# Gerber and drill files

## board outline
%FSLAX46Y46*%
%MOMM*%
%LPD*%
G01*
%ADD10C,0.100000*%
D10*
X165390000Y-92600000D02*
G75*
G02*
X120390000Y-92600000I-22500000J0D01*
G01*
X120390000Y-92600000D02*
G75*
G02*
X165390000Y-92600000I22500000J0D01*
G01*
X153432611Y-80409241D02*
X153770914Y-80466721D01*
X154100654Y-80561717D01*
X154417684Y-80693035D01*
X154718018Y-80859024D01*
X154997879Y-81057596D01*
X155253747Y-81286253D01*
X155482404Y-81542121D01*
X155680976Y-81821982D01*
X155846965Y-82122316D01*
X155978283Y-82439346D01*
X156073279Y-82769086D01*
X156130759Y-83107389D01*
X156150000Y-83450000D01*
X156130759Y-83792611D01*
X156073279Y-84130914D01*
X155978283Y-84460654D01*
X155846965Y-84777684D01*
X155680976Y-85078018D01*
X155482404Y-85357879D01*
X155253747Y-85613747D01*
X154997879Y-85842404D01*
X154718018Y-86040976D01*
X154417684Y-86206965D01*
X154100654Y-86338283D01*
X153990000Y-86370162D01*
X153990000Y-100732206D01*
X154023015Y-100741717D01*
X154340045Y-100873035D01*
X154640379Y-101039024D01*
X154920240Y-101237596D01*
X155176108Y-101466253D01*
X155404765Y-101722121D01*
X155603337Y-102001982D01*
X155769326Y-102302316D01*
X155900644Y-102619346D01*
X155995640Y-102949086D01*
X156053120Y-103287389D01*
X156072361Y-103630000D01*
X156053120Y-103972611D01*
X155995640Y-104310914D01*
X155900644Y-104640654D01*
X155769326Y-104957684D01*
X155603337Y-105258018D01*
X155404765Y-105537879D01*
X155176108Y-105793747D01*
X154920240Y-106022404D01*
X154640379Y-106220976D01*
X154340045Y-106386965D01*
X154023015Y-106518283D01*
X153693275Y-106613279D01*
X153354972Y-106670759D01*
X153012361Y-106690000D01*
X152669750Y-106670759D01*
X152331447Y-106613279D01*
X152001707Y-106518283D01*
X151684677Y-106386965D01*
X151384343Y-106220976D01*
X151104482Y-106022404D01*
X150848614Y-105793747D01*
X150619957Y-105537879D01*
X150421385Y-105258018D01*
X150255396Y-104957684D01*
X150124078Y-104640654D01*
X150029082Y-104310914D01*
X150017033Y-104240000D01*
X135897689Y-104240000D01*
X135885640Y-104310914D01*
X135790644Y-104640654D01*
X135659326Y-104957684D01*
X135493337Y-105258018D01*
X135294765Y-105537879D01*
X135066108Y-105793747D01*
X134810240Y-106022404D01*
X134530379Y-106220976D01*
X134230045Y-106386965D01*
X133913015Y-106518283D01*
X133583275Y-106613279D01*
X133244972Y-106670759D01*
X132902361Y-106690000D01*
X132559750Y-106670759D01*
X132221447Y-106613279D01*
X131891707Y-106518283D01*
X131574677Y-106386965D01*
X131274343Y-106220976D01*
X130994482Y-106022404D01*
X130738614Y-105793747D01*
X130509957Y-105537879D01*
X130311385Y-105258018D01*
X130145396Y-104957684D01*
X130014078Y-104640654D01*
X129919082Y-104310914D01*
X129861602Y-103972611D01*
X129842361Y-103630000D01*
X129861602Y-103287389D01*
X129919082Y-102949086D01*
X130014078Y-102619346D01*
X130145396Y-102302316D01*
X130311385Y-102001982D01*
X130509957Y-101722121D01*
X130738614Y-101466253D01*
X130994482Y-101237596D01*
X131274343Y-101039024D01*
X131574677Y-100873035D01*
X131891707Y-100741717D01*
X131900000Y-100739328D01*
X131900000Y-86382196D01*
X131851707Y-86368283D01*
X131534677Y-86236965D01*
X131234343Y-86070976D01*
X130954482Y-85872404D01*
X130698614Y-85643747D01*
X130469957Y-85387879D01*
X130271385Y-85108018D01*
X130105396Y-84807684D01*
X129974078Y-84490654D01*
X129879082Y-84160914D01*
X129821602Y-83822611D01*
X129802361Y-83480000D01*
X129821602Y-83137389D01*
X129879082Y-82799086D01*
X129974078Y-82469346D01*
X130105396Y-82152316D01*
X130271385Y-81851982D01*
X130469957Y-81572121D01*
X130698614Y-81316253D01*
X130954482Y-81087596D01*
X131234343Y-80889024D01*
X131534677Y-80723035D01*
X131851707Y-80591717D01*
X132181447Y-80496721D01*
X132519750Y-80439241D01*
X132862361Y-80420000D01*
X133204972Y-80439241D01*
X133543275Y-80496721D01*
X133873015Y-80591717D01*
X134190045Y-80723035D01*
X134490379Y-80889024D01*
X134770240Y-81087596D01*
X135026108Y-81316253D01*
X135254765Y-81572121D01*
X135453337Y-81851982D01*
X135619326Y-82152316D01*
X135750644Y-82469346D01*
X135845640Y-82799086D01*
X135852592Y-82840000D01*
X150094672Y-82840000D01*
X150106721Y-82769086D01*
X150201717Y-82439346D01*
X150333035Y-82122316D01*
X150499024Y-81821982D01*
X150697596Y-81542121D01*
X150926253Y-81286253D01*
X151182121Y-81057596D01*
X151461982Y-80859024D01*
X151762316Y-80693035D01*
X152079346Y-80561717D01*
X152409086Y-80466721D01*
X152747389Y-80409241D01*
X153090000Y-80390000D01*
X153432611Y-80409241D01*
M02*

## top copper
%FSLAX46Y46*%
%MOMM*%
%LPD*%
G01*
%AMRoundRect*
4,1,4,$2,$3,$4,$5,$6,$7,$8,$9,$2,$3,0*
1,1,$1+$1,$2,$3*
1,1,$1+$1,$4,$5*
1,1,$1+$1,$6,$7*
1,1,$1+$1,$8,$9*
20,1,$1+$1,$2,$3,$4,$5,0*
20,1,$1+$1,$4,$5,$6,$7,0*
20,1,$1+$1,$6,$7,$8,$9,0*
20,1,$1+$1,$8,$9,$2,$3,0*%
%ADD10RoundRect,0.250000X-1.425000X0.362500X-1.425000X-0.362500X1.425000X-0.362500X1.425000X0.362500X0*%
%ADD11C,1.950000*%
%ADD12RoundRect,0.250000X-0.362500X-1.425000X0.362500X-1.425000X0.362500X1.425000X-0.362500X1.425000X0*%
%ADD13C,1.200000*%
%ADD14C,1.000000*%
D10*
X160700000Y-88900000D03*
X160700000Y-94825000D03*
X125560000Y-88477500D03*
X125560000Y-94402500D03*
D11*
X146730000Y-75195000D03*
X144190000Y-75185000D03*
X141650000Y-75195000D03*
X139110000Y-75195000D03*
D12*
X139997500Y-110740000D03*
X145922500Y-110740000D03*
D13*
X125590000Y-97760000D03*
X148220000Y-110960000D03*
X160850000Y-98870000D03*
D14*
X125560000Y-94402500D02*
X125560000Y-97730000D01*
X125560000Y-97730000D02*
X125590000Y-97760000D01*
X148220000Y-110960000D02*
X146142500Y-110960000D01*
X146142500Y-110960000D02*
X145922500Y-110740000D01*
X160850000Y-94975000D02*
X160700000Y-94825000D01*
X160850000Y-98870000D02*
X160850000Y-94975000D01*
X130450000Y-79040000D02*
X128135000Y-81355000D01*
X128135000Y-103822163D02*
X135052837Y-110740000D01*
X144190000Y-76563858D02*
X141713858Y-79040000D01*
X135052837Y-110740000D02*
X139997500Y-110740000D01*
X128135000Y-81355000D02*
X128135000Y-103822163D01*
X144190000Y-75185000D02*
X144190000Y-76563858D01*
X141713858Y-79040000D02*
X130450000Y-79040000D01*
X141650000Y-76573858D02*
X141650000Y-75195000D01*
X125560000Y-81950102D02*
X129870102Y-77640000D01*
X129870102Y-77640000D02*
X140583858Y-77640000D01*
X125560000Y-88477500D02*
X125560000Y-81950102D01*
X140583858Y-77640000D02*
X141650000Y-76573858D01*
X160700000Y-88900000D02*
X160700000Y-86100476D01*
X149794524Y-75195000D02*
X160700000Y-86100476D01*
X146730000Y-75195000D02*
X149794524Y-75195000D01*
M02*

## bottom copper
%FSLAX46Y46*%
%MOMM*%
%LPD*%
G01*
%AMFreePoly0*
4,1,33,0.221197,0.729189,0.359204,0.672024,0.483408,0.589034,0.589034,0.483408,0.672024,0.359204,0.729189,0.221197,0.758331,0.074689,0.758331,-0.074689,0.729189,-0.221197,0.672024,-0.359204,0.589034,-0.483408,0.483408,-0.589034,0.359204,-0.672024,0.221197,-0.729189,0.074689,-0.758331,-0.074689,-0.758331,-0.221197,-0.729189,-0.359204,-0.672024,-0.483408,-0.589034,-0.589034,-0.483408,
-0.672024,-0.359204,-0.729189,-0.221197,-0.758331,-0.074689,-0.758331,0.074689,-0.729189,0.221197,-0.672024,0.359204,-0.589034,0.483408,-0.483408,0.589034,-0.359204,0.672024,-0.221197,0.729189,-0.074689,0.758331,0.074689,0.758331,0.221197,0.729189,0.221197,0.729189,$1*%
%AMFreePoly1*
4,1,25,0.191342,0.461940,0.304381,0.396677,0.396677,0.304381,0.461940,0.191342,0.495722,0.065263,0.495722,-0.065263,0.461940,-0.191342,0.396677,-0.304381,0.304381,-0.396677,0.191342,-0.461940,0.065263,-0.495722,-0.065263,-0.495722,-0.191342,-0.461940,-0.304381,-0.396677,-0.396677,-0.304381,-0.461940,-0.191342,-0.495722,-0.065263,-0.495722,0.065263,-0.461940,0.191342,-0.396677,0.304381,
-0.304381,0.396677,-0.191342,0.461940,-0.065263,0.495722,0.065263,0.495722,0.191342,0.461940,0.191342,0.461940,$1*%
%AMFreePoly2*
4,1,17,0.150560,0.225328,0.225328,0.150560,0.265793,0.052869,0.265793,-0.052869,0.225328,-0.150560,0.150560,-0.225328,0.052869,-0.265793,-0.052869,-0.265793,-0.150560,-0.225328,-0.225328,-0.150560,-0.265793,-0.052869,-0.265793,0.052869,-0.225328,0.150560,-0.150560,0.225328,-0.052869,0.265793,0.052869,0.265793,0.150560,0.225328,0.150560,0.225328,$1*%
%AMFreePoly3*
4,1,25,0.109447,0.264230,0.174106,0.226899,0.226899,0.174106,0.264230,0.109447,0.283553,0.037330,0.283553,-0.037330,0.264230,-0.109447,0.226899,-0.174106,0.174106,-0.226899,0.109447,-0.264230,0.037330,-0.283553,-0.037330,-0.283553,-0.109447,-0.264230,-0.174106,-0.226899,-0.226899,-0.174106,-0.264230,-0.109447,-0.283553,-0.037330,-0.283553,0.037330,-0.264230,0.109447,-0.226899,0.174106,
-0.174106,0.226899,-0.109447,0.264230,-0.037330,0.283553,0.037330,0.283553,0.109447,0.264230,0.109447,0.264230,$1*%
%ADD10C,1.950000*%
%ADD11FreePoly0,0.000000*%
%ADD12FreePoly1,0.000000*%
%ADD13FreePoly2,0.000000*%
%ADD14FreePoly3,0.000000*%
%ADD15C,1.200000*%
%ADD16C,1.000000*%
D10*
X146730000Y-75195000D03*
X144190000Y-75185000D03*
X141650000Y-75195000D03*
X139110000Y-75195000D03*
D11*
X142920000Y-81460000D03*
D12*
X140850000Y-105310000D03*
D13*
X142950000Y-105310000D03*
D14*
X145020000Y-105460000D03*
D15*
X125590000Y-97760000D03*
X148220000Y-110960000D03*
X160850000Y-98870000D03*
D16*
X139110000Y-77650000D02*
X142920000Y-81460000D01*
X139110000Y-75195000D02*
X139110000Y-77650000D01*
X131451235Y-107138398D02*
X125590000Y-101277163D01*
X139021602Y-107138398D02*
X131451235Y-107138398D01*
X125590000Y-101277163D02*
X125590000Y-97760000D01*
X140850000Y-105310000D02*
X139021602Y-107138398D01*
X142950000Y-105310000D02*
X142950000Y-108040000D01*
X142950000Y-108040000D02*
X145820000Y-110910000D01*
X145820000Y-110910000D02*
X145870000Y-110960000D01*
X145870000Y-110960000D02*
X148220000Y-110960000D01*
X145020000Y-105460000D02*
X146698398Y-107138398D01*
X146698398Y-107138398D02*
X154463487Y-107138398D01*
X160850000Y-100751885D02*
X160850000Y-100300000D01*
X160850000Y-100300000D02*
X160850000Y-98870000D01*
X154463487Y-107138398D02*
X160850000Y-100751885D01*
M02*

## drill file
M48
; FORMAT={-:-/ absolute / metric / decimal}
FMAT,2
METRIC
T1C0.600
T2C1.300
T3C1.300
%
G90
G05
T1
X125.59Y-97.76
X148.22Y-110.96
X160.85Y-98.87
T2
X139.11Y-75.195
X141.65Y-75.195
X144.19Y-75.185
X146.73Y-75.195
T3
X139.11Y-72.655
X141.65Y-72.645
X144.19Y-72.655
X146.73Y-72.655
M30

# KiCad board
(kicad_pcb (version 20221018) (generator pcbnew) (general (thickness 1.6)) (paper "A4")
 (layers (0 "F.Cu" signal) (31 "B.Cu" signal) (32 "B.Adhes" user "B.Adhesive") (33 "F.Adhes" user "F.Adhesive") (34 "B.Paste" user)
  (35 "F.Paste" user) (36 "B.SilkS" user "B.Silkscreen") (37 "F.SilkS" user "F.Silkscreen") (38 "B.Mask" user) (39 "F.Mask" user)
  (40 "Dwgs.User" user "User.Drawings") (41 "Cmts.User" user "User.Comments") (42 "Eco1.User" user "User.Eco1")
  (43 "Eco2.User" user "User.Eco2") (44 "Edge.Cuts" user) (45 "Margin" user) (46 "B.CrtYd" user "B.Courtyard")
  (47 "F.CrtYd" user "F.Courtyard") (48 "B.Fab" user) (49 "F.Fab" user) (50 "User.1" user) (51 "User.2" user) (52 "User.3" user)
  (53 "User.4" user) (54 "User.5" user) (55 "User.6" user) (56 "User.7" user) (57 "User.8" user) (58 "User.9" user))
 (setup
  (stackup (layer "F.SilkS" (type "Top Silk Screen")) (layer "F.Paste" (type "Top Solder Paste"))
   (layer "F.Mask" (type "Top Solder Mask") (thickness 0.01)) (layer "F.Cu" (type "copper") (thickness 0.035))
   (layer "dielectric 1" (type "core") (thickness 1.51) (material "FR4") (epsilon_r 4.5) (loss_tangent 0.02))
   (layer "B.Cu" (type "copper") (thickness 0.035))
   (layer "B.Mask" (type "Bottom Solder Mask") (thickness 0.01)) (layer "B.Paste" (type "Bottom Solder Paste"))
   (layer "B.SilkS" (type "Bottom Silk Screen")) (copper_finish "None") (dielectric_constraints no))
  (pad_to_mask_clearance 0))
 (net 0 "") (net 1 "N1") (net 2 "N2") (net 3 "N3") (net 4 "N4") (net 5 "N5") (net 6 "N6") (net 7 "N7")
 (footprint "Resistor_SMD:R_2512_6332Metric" (layer "F.Cu") (at 160.7 91.8625 -90)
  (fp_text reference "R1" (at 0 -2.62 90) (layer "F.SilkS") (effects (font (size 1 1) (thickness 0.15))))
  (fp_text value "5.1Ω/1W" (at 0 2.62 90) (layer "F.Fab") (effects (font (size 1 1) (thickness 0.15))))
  (pad "1" smd roundrect (at -2.9625 0 270) (size 1.225 3.35) (layers "F.Cu" "F.Paste" "F.Mask") (roundrect_rratio 0.2040816327)
   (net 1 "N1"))
  (pad "2" smd roundrect (at 2.9625 0 270) (size 1.225 3.35) (layers "F.Cu" "F.Paste" "F.Mask") (roundrect_rratio 0.2040816327) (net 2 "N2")))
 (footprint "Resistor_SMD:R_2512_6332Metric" (layer "F.Cu") (at 125.56 91.44 -90)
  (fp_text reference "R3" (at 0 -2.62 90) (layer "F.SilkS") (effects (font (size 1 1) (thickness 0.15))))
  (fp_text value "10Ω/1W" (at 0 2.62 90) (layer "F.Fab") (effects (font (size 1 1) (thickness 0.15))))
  (pad "1" smd roundrect (at -2.9625 0 270) (size 1.225 3.35) (layers "F.Cu" "F.Paste" "F.Mask") (roundrect_rratio 0.2040816327)
   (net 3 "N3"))
  (pad "2" smd roundrect (at 2.9625 0 270) (size 1.225 3.35) (layers "F.Cu" "F.Paste" "F.Mask") (roundrect_rratio 0.2040816327) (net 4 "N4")))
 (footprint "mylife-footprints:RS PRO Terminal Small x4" (layer "F.Cu") (at 146.73 75.195 180)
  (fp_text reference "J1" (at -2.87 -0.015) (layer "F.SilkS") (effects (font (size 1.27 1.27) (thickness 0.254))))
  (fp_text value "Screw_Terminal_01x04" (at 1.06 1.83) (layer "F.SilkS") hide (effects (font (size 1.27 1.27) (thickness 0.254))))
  (pad "" np_thru_hole circle (at 0 2.54 180) (size 1.3 1.3) (drill 1.3) (layers "*.Cu" "*.Mask"))
  (pad "" np_thru_hole circle (at 2.54 2.54 180) (size 1.3 1.3) (drill 1.3) (layers "*.Cu" "*.Mask"))
  (pad "" np_thru_hole circle (at 5.08 2.55 180) (size 1.3 1.3) (drill 1.3) (layers "*.Cu" "*.Mask"))
  (pad "" np_thru_hole circle (at 7.62 2.54 180) (size 1.3 1.3) (drill 1.3) (layers "*.Cu" "*.Mask"))
  (pad "1" thru_hole circle (at 0 0 180) (size 1.95 1.95) (drill 1.3) (layers "*.Cu" "*.Mask") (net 1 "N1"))
  (pad "2" thru_hole circle (at 2.54 0.01 180) (size 1.95 1.95) (drill 1.3) (layers "*.Cu" "*.Mask") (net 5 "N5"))
  (pad "3" thru_hole circle (at 5.08 0 180) (size 1.95 1.95) (drill 1.3) (layers "*.Cu" "*.Mask") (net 3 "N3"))
  (pad "4" thru_hole circle (at 7.62 0 180) (size 1.95 1.95) (drill 1.3) (layers "*.Cu" "*.Mask") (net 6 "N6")))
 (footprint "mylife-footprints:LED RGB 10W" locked (layer "F.Cu") (at 142.94 92.59)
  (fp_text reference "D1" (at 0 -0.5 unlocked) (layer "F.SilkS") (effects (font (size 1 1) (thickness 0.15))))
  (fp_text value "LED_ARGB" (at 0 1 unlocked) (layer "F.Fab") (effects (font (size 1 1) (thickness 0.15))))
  (fp_poly
   (pts (xy 10.492611 -12.180759) (xy 10.830914 -12.123279) (xy 11.160654 -12.028283) (xy 11.477684 -11.896965) (xy 11.778018 -11.730976)
    (xy 12.057879 -11.532404) (xy 12.313747 -11.303747) (xy 12.542404 -11.047879) (xy 12.740976 -10.768018) (xy 12.906965 -10.467684)
    (xy 13.038283 -10.150654) (xy 13.133279 -9.820914) (xy 13.190759 -9.482611) (xy 13.21 -9.14) (xy 13.190759 -8.797389)
    (xy 13.133279 -8.459086) (xy 13.038283 -8.129346) (xy 12.906965 -7.812316) (xy 12.740976 -7.511982) (xy 12.542404 -7.232121)
    (xy 12.313747 -6.976253) (xy 12.057879 -6.747596) (xy 11.778018 -6.549024) (xy 11.477684 -6.383035) (xy 11.160654 -6.251717)
    (xy 11.05 -6.219838) (xy 11.05 8.142206) (xy 11.083015 8.151717) (xy 11.400045 8.283035) (xy 11.700379 8.449024) (xy 11.98024 8.647596)
    (xy 12.236108 8.876253) (xy 12.464765 9.132121) (xy 12.663337 9.411982) (xy 12.829326 9.712316) (xy 12.960644 10.029346)
    (xy 13.05564 10.359086) (xy 13.11312 10.697389) (xy 13.132361 11.04) (xy 13.11312 11.382611) (xy 13.05564 11.720914)
    (xy 12.960644 12.050654) (xy 12.829326 12.367684) (xy 12.663337 12.668018) (xy 12.464765 12.947879) (xy 12.236108 13.203747)
    (xy 11.98024 13.432404) (xy 11.700379 13.630976) (xy 11.400045 13.796965) (xy 11.083015 13.928283) (xy 10.753275 14.023279)
    (xy 10.414972 14.080759) (xy 10.072361 14.1) (xy 9.72975 14.080759) (xy 9.391447 14.023279) (xy 9.061707 13.928283)
    (xy 8.744677 13.796965) (xy 8.444343 13.630976) (xy 8.164482 13.432404) (xy 7.908614 13.203747) (xy 7.679957 12.947879)
    (xy 7.481385 12.668018) (xy 7.315396 12.367684) (xy 7.184078 12.050654) (xy 7.089082 11.720914) (xy 7.077033 11.65) (xy -7.042311 11.65)
    (xy -7.05436 11.720914) (xy -7.149356 12.050654) (xy -7.280674 12.367684) (xy -7.446663 12.668018) (xy -7.645235 12.947879)
    (xy -7.873892 13.203747) (xy -8.12976 13.432404) (xy -8.409621 13.630976) (xy -8.709955 13.796965) (xy -9.026985 13.928283)
    (xy -9.356725 14.023279) (xy -9.695028 14.080759) (xy -10.037639 14.1) (xy -10.38025 14.080759) (xy -10.718553 14.023279)
    (xy -11.048293 13.928283) (xy -11.365323 13.796965) (xy -11.665657 13.630976) (xy -11.945518 13.432404) (xy -12.201386 13.203747)
    (xy -12.430043 12.947879) (xy -12.628615 12.668018) (xy -12.794604 12.367684) (xy -12.925922 12.050654) (xy -13.020918 11.720914)
    (xy -13.078398 11.382611) (xy -13.097639 11.04) (xy -13.078398 10.697389) (xy -13.020918 10.359086) (xy -12.925922 10.029346)
    (xy -12.794604 9.712316) (xy -12.628615 9.411982) (xy -12.430043 9.132121) (xy -12.201386 8.876253) (xy -11.945518 8.647596)
    (xy -11.665657 8.449024) (xy -11.365323 8.283035) (xy -11.048293 8.151717) (xy -11.04 8.149328) (xy -11.04 -6.207804)
    (xy -11.088293 -6.221717) (xy -11.405323 -6.353035) (xy -11.705657 -6.519024) (xy -11.985518 -6.717596) (xy -12.241386 -6.946253)
    (xy -12.470043 -7.202121) (xy -12.668615 -7.481982) (xy -12.834604 -7.782316) (xy -12.965922 -8.099346) (xy -13.060918 -8.429086)
    (xy -13.118398 -8.767389) (xy -13.137639 -9.11) (xy -13.118398 -9.452611) (xy -13.060918 -9.790914) (xy -12.965922 -10.120654)
    (xy -12.834604 -10.437684) (xy -12.668615 -10.738018) (xy -12.470043 -11.017879) (xy -12.241386 -11.273747) (xy -11.985518 -11.502404)
    (xy -11.705657 -11.700976) (xy -11.405323 -11.866965) (xy -11.088293 -11.998283) (xy -10.758553 -12.093279) (xy -10.42025 -12.150759)
    (xy -10.077639 -12.17) (xy -9.735028 -12.150759) (xy -9.396725 -12.093279) (xy -9.066985 -11.998283) (xy -8.749955 -11.866965)
    (xy -8.449621 -11.700976) (xy -8.16976 -11.502404) (xy -7.913892 -11.273747) (xy -7.685235 -11.017879) (xy -7.486663 -10.738018)
    (xy -7.320674 -10.437684) (xy -7.189356 -10.120654) (xy -7.09436 -9.790914) (xy -7.087408 -9.75) (xy 7.154672 -9.75)
    (xy 7.166721 -9.820914) (xy 7.261717 -10.150654) (xy 7.393035 -10.467684) (xy 7.559024 -10.768018) (xy 7.757596 -11.047879)
    (xy 7.986253 -11.303747) (xy 8.242121 -11.532404) (xy 8.521982 -11.730976) (xy 8.822316 -11.896965) (xy 9.139346 -12.028283)
    (xy 9.469086 -12.123279) (xy 9.807389 -12.180759) (xy 10.15 -12.2))
   (stroke (width 0.1) (type solid)) (fill none) (layer "Edge.Cuts"))
  (pad "1" smd custom locked (at -0.02 -11.13) (size 1.524 1.524) (layers "B.Cu" "B.Paste" "B.Mask") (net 6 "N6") (thermal_bridge_angle 45)
   (options (clearance outline) (anchor circle)) (primitives))
  (pad "2" smd custom locked (at -2.09 12.72) (size 1 1) (layers "B.Cu" "B.Paste" "B.Mask") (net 4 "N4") (thermal_bridge_angle 45)
   (options (clearance outline) (anchor circle)) (primitives))
  (pad "3" smd custom locked (at 0.01 12.72) (size 0.542 0.542) (layers "B.Cu" "B.Paste" "B.Mask") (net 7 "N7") (thermal_bridge_angle 45)
   (options (clearance outline) (anchor circle)) (primitives))
  (pad "4" smd custom locked (at 2.08 12.87) (size 0.572 0.572) (layers "B.Cu" "B.Paste" "B.Mask") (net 2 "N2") (thermal_bridge_angle 45)
   (options (clearance outline) (anchor circle)) (primitives)))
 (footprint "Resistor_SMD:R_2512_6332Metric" (layer "F.Cu") (at 142.96 110.74)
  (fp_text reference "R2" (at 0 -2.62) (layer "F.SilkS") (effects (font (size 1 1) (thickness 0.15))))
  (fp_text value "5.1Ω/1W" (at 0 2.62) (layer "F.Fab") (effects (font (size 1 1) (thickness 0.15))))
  (pad "1" smd roundrect (at -2.9625 0) (size 1.225 3.35) (layers "F.Cu" "F.Paste" "F.Mask") (roundrect_rratio 0.2040816327) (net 5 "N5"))
  (pad "2" smd roundrect (at 2.9625 0) (size 1.225 3.35) (layers "F.Cu" "F.Paste" "F.Mask") (roundrect_rratio 0.2040816327) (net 7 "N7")))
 (gr_circle locked (center 142.89 92.6) (end 165.39 92.6) (stroke (width 0.1) (type default)) (fill none) (layer "Edge.Cuts"))
 (segment (start 139.11 77.65) (end 142.92 81.46) (width 1) (layer "B.Cu") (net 6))
 (segment (start 139.11 75.195) (end 139.11 77.65) (width 1) (layer "B.Cu") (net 6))
 (segment (start 125.56 94.4025) (end 125.56 97.73) (width 1) (layer "F.Cu") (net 4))
 (segment (start 125.56 97.73) (end 125.59 97.76) (width 1) (layer "F.Cu") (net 4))
 (via (at 125.59 97.76) (size 1.2) (drill 0.6) (layers "F.Cu" "B.Cu") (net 4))
 (segment (start 131.451235 107.138398) (end 125.59 101.277163) (width 1) (layer "B.Cu") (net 4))
 (segment (start 139.021602 107.138398) (end 131.451235 107.138398) (width 1) (layer "B.Cu") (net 4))
 (segment (start 125.59 101.277163) (end 125.59 97.76) (width 1) (layer "B.Cu") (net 4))
 (segment (start 140.85 105.31) (end 139.021602 107.138398) (width 1) (layer "B.Cu") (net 4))
 (segment (start 148.22 110.96) (end 146.1425 110.96) (width 1) (layer "F.Cu") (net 7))
 (segment (start 146.1425 110.96) (end 145.9225 110.74) (width 1) (layer "F.Cu") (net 7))
 (via (at 148.22 110.96) (size 1.2) (drill 0.6) (layers "F.Cu" "B.Cu") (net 7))
 (segment (start 142.95 105.31) (end 142.95 108.04) (width 1) (layer "B.Cu") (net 7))
 (segment (start 142.95 108.04) (end 145.82 110.91) (width 1) (layer "B.Cu") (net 7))
 (segment (start 145.82 110.91) (end 145.87 110.96) (width 1) (layer "B.Cu") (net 7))
 (segment (start 145.87 110.96) (end 148.22 110.96) (width 1) (layer "B.Cu") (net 7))
 (segment (start 160.85 94.975) (end 160.7 94.825) (width 1) (layer "F.Cu") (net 2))
 (segment (start 160.85 98.87) (end 160.85 94.975) (width 1) (layer "F.Cu") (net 2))
 (via (at 160.85 98.87) (size 1.2) (drill 0.6) (layers "F.Cu" "B.Cu") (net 2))
 (segment (start 145.02 105.46) (end 146.698398 107.138398) (width 1) (layer "B.Cu") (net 2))
 (segment (start 146.698398 107.138398) (end 154.463487 107.138398) (width 1) (layer "B.Cu") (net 2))
 (segment (start 160.85 100.751885) (end 160.85 100.3) (width 1) (layer "B.Cu") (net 2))
 (segment (start 160.85 100.3) (end 160.85 98.87) (width 1) (layer "B.Cu") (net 2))
 (segment (start 154.463487 107.138398) (end 160.85 100.751885) (width 1) (layer "B.Cu") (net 2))
 (segment (start 130.45 79.04) (end 128.135 81.355) (width 1) (layer "F.Cu") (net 5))
 (segment (start 128.135 103.822163) (end 135.052837 110.74) (width 1) (layer "F.Cu") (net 5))
 (segment (start 144.19 76.563858) (end 141.713858 79.04) (width 1) (layer "F.Cu") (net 5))
 (segment (start 135.052837 110.74) (end 139.9975 110.74) (width 1) (layer "F.Cu") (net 5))
 (segment (start 128.135 81.355) (end 128.135 103.822163) (width 1) (layer "F.Cu") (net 5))
 (segment (start 144.19 75.185) (end 144.19 76.563858) (width 1) (layer "F.Cu") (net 5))
 (segment (start 141.713858 79.04) (end 130.45 79.04) (width 1) (layer "F.Cu") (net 5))
 (segment (start 141.65 76.573858) (end 141.65 75.195) (width 1) (layer "F.Cu") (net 3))
 (segment (start 125.56 81.950102) (end 129.870102 77.64) (width 1) (layer "F.Cu") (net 3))
 (segment (start 129.870102 77.64) (end 140.583858 77.64) (width 1) (layer "F.Cu") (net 3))
 (segment (start 125.56 88.4775) (end 125.56 81.950102) (width 1) (layer "F.Cu") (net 3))
 (segment (start 140.583858 77.64) (end 141.65 76.573858) (width 1) (layer "F.Cu") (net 3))
 (segment (start 160.7 88.9) (end 160.7 86.100476) (width 1) (layer "F.Cu") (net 1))
 (segment (start 149.794524 75.195) (end 160.7 86.100476) (width 1) (layer "F.Cu") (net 1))
 (segment (start 146.73 75.195) (end 149.794524 75.195) (width 1) (layer "F.Cu") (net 1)))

